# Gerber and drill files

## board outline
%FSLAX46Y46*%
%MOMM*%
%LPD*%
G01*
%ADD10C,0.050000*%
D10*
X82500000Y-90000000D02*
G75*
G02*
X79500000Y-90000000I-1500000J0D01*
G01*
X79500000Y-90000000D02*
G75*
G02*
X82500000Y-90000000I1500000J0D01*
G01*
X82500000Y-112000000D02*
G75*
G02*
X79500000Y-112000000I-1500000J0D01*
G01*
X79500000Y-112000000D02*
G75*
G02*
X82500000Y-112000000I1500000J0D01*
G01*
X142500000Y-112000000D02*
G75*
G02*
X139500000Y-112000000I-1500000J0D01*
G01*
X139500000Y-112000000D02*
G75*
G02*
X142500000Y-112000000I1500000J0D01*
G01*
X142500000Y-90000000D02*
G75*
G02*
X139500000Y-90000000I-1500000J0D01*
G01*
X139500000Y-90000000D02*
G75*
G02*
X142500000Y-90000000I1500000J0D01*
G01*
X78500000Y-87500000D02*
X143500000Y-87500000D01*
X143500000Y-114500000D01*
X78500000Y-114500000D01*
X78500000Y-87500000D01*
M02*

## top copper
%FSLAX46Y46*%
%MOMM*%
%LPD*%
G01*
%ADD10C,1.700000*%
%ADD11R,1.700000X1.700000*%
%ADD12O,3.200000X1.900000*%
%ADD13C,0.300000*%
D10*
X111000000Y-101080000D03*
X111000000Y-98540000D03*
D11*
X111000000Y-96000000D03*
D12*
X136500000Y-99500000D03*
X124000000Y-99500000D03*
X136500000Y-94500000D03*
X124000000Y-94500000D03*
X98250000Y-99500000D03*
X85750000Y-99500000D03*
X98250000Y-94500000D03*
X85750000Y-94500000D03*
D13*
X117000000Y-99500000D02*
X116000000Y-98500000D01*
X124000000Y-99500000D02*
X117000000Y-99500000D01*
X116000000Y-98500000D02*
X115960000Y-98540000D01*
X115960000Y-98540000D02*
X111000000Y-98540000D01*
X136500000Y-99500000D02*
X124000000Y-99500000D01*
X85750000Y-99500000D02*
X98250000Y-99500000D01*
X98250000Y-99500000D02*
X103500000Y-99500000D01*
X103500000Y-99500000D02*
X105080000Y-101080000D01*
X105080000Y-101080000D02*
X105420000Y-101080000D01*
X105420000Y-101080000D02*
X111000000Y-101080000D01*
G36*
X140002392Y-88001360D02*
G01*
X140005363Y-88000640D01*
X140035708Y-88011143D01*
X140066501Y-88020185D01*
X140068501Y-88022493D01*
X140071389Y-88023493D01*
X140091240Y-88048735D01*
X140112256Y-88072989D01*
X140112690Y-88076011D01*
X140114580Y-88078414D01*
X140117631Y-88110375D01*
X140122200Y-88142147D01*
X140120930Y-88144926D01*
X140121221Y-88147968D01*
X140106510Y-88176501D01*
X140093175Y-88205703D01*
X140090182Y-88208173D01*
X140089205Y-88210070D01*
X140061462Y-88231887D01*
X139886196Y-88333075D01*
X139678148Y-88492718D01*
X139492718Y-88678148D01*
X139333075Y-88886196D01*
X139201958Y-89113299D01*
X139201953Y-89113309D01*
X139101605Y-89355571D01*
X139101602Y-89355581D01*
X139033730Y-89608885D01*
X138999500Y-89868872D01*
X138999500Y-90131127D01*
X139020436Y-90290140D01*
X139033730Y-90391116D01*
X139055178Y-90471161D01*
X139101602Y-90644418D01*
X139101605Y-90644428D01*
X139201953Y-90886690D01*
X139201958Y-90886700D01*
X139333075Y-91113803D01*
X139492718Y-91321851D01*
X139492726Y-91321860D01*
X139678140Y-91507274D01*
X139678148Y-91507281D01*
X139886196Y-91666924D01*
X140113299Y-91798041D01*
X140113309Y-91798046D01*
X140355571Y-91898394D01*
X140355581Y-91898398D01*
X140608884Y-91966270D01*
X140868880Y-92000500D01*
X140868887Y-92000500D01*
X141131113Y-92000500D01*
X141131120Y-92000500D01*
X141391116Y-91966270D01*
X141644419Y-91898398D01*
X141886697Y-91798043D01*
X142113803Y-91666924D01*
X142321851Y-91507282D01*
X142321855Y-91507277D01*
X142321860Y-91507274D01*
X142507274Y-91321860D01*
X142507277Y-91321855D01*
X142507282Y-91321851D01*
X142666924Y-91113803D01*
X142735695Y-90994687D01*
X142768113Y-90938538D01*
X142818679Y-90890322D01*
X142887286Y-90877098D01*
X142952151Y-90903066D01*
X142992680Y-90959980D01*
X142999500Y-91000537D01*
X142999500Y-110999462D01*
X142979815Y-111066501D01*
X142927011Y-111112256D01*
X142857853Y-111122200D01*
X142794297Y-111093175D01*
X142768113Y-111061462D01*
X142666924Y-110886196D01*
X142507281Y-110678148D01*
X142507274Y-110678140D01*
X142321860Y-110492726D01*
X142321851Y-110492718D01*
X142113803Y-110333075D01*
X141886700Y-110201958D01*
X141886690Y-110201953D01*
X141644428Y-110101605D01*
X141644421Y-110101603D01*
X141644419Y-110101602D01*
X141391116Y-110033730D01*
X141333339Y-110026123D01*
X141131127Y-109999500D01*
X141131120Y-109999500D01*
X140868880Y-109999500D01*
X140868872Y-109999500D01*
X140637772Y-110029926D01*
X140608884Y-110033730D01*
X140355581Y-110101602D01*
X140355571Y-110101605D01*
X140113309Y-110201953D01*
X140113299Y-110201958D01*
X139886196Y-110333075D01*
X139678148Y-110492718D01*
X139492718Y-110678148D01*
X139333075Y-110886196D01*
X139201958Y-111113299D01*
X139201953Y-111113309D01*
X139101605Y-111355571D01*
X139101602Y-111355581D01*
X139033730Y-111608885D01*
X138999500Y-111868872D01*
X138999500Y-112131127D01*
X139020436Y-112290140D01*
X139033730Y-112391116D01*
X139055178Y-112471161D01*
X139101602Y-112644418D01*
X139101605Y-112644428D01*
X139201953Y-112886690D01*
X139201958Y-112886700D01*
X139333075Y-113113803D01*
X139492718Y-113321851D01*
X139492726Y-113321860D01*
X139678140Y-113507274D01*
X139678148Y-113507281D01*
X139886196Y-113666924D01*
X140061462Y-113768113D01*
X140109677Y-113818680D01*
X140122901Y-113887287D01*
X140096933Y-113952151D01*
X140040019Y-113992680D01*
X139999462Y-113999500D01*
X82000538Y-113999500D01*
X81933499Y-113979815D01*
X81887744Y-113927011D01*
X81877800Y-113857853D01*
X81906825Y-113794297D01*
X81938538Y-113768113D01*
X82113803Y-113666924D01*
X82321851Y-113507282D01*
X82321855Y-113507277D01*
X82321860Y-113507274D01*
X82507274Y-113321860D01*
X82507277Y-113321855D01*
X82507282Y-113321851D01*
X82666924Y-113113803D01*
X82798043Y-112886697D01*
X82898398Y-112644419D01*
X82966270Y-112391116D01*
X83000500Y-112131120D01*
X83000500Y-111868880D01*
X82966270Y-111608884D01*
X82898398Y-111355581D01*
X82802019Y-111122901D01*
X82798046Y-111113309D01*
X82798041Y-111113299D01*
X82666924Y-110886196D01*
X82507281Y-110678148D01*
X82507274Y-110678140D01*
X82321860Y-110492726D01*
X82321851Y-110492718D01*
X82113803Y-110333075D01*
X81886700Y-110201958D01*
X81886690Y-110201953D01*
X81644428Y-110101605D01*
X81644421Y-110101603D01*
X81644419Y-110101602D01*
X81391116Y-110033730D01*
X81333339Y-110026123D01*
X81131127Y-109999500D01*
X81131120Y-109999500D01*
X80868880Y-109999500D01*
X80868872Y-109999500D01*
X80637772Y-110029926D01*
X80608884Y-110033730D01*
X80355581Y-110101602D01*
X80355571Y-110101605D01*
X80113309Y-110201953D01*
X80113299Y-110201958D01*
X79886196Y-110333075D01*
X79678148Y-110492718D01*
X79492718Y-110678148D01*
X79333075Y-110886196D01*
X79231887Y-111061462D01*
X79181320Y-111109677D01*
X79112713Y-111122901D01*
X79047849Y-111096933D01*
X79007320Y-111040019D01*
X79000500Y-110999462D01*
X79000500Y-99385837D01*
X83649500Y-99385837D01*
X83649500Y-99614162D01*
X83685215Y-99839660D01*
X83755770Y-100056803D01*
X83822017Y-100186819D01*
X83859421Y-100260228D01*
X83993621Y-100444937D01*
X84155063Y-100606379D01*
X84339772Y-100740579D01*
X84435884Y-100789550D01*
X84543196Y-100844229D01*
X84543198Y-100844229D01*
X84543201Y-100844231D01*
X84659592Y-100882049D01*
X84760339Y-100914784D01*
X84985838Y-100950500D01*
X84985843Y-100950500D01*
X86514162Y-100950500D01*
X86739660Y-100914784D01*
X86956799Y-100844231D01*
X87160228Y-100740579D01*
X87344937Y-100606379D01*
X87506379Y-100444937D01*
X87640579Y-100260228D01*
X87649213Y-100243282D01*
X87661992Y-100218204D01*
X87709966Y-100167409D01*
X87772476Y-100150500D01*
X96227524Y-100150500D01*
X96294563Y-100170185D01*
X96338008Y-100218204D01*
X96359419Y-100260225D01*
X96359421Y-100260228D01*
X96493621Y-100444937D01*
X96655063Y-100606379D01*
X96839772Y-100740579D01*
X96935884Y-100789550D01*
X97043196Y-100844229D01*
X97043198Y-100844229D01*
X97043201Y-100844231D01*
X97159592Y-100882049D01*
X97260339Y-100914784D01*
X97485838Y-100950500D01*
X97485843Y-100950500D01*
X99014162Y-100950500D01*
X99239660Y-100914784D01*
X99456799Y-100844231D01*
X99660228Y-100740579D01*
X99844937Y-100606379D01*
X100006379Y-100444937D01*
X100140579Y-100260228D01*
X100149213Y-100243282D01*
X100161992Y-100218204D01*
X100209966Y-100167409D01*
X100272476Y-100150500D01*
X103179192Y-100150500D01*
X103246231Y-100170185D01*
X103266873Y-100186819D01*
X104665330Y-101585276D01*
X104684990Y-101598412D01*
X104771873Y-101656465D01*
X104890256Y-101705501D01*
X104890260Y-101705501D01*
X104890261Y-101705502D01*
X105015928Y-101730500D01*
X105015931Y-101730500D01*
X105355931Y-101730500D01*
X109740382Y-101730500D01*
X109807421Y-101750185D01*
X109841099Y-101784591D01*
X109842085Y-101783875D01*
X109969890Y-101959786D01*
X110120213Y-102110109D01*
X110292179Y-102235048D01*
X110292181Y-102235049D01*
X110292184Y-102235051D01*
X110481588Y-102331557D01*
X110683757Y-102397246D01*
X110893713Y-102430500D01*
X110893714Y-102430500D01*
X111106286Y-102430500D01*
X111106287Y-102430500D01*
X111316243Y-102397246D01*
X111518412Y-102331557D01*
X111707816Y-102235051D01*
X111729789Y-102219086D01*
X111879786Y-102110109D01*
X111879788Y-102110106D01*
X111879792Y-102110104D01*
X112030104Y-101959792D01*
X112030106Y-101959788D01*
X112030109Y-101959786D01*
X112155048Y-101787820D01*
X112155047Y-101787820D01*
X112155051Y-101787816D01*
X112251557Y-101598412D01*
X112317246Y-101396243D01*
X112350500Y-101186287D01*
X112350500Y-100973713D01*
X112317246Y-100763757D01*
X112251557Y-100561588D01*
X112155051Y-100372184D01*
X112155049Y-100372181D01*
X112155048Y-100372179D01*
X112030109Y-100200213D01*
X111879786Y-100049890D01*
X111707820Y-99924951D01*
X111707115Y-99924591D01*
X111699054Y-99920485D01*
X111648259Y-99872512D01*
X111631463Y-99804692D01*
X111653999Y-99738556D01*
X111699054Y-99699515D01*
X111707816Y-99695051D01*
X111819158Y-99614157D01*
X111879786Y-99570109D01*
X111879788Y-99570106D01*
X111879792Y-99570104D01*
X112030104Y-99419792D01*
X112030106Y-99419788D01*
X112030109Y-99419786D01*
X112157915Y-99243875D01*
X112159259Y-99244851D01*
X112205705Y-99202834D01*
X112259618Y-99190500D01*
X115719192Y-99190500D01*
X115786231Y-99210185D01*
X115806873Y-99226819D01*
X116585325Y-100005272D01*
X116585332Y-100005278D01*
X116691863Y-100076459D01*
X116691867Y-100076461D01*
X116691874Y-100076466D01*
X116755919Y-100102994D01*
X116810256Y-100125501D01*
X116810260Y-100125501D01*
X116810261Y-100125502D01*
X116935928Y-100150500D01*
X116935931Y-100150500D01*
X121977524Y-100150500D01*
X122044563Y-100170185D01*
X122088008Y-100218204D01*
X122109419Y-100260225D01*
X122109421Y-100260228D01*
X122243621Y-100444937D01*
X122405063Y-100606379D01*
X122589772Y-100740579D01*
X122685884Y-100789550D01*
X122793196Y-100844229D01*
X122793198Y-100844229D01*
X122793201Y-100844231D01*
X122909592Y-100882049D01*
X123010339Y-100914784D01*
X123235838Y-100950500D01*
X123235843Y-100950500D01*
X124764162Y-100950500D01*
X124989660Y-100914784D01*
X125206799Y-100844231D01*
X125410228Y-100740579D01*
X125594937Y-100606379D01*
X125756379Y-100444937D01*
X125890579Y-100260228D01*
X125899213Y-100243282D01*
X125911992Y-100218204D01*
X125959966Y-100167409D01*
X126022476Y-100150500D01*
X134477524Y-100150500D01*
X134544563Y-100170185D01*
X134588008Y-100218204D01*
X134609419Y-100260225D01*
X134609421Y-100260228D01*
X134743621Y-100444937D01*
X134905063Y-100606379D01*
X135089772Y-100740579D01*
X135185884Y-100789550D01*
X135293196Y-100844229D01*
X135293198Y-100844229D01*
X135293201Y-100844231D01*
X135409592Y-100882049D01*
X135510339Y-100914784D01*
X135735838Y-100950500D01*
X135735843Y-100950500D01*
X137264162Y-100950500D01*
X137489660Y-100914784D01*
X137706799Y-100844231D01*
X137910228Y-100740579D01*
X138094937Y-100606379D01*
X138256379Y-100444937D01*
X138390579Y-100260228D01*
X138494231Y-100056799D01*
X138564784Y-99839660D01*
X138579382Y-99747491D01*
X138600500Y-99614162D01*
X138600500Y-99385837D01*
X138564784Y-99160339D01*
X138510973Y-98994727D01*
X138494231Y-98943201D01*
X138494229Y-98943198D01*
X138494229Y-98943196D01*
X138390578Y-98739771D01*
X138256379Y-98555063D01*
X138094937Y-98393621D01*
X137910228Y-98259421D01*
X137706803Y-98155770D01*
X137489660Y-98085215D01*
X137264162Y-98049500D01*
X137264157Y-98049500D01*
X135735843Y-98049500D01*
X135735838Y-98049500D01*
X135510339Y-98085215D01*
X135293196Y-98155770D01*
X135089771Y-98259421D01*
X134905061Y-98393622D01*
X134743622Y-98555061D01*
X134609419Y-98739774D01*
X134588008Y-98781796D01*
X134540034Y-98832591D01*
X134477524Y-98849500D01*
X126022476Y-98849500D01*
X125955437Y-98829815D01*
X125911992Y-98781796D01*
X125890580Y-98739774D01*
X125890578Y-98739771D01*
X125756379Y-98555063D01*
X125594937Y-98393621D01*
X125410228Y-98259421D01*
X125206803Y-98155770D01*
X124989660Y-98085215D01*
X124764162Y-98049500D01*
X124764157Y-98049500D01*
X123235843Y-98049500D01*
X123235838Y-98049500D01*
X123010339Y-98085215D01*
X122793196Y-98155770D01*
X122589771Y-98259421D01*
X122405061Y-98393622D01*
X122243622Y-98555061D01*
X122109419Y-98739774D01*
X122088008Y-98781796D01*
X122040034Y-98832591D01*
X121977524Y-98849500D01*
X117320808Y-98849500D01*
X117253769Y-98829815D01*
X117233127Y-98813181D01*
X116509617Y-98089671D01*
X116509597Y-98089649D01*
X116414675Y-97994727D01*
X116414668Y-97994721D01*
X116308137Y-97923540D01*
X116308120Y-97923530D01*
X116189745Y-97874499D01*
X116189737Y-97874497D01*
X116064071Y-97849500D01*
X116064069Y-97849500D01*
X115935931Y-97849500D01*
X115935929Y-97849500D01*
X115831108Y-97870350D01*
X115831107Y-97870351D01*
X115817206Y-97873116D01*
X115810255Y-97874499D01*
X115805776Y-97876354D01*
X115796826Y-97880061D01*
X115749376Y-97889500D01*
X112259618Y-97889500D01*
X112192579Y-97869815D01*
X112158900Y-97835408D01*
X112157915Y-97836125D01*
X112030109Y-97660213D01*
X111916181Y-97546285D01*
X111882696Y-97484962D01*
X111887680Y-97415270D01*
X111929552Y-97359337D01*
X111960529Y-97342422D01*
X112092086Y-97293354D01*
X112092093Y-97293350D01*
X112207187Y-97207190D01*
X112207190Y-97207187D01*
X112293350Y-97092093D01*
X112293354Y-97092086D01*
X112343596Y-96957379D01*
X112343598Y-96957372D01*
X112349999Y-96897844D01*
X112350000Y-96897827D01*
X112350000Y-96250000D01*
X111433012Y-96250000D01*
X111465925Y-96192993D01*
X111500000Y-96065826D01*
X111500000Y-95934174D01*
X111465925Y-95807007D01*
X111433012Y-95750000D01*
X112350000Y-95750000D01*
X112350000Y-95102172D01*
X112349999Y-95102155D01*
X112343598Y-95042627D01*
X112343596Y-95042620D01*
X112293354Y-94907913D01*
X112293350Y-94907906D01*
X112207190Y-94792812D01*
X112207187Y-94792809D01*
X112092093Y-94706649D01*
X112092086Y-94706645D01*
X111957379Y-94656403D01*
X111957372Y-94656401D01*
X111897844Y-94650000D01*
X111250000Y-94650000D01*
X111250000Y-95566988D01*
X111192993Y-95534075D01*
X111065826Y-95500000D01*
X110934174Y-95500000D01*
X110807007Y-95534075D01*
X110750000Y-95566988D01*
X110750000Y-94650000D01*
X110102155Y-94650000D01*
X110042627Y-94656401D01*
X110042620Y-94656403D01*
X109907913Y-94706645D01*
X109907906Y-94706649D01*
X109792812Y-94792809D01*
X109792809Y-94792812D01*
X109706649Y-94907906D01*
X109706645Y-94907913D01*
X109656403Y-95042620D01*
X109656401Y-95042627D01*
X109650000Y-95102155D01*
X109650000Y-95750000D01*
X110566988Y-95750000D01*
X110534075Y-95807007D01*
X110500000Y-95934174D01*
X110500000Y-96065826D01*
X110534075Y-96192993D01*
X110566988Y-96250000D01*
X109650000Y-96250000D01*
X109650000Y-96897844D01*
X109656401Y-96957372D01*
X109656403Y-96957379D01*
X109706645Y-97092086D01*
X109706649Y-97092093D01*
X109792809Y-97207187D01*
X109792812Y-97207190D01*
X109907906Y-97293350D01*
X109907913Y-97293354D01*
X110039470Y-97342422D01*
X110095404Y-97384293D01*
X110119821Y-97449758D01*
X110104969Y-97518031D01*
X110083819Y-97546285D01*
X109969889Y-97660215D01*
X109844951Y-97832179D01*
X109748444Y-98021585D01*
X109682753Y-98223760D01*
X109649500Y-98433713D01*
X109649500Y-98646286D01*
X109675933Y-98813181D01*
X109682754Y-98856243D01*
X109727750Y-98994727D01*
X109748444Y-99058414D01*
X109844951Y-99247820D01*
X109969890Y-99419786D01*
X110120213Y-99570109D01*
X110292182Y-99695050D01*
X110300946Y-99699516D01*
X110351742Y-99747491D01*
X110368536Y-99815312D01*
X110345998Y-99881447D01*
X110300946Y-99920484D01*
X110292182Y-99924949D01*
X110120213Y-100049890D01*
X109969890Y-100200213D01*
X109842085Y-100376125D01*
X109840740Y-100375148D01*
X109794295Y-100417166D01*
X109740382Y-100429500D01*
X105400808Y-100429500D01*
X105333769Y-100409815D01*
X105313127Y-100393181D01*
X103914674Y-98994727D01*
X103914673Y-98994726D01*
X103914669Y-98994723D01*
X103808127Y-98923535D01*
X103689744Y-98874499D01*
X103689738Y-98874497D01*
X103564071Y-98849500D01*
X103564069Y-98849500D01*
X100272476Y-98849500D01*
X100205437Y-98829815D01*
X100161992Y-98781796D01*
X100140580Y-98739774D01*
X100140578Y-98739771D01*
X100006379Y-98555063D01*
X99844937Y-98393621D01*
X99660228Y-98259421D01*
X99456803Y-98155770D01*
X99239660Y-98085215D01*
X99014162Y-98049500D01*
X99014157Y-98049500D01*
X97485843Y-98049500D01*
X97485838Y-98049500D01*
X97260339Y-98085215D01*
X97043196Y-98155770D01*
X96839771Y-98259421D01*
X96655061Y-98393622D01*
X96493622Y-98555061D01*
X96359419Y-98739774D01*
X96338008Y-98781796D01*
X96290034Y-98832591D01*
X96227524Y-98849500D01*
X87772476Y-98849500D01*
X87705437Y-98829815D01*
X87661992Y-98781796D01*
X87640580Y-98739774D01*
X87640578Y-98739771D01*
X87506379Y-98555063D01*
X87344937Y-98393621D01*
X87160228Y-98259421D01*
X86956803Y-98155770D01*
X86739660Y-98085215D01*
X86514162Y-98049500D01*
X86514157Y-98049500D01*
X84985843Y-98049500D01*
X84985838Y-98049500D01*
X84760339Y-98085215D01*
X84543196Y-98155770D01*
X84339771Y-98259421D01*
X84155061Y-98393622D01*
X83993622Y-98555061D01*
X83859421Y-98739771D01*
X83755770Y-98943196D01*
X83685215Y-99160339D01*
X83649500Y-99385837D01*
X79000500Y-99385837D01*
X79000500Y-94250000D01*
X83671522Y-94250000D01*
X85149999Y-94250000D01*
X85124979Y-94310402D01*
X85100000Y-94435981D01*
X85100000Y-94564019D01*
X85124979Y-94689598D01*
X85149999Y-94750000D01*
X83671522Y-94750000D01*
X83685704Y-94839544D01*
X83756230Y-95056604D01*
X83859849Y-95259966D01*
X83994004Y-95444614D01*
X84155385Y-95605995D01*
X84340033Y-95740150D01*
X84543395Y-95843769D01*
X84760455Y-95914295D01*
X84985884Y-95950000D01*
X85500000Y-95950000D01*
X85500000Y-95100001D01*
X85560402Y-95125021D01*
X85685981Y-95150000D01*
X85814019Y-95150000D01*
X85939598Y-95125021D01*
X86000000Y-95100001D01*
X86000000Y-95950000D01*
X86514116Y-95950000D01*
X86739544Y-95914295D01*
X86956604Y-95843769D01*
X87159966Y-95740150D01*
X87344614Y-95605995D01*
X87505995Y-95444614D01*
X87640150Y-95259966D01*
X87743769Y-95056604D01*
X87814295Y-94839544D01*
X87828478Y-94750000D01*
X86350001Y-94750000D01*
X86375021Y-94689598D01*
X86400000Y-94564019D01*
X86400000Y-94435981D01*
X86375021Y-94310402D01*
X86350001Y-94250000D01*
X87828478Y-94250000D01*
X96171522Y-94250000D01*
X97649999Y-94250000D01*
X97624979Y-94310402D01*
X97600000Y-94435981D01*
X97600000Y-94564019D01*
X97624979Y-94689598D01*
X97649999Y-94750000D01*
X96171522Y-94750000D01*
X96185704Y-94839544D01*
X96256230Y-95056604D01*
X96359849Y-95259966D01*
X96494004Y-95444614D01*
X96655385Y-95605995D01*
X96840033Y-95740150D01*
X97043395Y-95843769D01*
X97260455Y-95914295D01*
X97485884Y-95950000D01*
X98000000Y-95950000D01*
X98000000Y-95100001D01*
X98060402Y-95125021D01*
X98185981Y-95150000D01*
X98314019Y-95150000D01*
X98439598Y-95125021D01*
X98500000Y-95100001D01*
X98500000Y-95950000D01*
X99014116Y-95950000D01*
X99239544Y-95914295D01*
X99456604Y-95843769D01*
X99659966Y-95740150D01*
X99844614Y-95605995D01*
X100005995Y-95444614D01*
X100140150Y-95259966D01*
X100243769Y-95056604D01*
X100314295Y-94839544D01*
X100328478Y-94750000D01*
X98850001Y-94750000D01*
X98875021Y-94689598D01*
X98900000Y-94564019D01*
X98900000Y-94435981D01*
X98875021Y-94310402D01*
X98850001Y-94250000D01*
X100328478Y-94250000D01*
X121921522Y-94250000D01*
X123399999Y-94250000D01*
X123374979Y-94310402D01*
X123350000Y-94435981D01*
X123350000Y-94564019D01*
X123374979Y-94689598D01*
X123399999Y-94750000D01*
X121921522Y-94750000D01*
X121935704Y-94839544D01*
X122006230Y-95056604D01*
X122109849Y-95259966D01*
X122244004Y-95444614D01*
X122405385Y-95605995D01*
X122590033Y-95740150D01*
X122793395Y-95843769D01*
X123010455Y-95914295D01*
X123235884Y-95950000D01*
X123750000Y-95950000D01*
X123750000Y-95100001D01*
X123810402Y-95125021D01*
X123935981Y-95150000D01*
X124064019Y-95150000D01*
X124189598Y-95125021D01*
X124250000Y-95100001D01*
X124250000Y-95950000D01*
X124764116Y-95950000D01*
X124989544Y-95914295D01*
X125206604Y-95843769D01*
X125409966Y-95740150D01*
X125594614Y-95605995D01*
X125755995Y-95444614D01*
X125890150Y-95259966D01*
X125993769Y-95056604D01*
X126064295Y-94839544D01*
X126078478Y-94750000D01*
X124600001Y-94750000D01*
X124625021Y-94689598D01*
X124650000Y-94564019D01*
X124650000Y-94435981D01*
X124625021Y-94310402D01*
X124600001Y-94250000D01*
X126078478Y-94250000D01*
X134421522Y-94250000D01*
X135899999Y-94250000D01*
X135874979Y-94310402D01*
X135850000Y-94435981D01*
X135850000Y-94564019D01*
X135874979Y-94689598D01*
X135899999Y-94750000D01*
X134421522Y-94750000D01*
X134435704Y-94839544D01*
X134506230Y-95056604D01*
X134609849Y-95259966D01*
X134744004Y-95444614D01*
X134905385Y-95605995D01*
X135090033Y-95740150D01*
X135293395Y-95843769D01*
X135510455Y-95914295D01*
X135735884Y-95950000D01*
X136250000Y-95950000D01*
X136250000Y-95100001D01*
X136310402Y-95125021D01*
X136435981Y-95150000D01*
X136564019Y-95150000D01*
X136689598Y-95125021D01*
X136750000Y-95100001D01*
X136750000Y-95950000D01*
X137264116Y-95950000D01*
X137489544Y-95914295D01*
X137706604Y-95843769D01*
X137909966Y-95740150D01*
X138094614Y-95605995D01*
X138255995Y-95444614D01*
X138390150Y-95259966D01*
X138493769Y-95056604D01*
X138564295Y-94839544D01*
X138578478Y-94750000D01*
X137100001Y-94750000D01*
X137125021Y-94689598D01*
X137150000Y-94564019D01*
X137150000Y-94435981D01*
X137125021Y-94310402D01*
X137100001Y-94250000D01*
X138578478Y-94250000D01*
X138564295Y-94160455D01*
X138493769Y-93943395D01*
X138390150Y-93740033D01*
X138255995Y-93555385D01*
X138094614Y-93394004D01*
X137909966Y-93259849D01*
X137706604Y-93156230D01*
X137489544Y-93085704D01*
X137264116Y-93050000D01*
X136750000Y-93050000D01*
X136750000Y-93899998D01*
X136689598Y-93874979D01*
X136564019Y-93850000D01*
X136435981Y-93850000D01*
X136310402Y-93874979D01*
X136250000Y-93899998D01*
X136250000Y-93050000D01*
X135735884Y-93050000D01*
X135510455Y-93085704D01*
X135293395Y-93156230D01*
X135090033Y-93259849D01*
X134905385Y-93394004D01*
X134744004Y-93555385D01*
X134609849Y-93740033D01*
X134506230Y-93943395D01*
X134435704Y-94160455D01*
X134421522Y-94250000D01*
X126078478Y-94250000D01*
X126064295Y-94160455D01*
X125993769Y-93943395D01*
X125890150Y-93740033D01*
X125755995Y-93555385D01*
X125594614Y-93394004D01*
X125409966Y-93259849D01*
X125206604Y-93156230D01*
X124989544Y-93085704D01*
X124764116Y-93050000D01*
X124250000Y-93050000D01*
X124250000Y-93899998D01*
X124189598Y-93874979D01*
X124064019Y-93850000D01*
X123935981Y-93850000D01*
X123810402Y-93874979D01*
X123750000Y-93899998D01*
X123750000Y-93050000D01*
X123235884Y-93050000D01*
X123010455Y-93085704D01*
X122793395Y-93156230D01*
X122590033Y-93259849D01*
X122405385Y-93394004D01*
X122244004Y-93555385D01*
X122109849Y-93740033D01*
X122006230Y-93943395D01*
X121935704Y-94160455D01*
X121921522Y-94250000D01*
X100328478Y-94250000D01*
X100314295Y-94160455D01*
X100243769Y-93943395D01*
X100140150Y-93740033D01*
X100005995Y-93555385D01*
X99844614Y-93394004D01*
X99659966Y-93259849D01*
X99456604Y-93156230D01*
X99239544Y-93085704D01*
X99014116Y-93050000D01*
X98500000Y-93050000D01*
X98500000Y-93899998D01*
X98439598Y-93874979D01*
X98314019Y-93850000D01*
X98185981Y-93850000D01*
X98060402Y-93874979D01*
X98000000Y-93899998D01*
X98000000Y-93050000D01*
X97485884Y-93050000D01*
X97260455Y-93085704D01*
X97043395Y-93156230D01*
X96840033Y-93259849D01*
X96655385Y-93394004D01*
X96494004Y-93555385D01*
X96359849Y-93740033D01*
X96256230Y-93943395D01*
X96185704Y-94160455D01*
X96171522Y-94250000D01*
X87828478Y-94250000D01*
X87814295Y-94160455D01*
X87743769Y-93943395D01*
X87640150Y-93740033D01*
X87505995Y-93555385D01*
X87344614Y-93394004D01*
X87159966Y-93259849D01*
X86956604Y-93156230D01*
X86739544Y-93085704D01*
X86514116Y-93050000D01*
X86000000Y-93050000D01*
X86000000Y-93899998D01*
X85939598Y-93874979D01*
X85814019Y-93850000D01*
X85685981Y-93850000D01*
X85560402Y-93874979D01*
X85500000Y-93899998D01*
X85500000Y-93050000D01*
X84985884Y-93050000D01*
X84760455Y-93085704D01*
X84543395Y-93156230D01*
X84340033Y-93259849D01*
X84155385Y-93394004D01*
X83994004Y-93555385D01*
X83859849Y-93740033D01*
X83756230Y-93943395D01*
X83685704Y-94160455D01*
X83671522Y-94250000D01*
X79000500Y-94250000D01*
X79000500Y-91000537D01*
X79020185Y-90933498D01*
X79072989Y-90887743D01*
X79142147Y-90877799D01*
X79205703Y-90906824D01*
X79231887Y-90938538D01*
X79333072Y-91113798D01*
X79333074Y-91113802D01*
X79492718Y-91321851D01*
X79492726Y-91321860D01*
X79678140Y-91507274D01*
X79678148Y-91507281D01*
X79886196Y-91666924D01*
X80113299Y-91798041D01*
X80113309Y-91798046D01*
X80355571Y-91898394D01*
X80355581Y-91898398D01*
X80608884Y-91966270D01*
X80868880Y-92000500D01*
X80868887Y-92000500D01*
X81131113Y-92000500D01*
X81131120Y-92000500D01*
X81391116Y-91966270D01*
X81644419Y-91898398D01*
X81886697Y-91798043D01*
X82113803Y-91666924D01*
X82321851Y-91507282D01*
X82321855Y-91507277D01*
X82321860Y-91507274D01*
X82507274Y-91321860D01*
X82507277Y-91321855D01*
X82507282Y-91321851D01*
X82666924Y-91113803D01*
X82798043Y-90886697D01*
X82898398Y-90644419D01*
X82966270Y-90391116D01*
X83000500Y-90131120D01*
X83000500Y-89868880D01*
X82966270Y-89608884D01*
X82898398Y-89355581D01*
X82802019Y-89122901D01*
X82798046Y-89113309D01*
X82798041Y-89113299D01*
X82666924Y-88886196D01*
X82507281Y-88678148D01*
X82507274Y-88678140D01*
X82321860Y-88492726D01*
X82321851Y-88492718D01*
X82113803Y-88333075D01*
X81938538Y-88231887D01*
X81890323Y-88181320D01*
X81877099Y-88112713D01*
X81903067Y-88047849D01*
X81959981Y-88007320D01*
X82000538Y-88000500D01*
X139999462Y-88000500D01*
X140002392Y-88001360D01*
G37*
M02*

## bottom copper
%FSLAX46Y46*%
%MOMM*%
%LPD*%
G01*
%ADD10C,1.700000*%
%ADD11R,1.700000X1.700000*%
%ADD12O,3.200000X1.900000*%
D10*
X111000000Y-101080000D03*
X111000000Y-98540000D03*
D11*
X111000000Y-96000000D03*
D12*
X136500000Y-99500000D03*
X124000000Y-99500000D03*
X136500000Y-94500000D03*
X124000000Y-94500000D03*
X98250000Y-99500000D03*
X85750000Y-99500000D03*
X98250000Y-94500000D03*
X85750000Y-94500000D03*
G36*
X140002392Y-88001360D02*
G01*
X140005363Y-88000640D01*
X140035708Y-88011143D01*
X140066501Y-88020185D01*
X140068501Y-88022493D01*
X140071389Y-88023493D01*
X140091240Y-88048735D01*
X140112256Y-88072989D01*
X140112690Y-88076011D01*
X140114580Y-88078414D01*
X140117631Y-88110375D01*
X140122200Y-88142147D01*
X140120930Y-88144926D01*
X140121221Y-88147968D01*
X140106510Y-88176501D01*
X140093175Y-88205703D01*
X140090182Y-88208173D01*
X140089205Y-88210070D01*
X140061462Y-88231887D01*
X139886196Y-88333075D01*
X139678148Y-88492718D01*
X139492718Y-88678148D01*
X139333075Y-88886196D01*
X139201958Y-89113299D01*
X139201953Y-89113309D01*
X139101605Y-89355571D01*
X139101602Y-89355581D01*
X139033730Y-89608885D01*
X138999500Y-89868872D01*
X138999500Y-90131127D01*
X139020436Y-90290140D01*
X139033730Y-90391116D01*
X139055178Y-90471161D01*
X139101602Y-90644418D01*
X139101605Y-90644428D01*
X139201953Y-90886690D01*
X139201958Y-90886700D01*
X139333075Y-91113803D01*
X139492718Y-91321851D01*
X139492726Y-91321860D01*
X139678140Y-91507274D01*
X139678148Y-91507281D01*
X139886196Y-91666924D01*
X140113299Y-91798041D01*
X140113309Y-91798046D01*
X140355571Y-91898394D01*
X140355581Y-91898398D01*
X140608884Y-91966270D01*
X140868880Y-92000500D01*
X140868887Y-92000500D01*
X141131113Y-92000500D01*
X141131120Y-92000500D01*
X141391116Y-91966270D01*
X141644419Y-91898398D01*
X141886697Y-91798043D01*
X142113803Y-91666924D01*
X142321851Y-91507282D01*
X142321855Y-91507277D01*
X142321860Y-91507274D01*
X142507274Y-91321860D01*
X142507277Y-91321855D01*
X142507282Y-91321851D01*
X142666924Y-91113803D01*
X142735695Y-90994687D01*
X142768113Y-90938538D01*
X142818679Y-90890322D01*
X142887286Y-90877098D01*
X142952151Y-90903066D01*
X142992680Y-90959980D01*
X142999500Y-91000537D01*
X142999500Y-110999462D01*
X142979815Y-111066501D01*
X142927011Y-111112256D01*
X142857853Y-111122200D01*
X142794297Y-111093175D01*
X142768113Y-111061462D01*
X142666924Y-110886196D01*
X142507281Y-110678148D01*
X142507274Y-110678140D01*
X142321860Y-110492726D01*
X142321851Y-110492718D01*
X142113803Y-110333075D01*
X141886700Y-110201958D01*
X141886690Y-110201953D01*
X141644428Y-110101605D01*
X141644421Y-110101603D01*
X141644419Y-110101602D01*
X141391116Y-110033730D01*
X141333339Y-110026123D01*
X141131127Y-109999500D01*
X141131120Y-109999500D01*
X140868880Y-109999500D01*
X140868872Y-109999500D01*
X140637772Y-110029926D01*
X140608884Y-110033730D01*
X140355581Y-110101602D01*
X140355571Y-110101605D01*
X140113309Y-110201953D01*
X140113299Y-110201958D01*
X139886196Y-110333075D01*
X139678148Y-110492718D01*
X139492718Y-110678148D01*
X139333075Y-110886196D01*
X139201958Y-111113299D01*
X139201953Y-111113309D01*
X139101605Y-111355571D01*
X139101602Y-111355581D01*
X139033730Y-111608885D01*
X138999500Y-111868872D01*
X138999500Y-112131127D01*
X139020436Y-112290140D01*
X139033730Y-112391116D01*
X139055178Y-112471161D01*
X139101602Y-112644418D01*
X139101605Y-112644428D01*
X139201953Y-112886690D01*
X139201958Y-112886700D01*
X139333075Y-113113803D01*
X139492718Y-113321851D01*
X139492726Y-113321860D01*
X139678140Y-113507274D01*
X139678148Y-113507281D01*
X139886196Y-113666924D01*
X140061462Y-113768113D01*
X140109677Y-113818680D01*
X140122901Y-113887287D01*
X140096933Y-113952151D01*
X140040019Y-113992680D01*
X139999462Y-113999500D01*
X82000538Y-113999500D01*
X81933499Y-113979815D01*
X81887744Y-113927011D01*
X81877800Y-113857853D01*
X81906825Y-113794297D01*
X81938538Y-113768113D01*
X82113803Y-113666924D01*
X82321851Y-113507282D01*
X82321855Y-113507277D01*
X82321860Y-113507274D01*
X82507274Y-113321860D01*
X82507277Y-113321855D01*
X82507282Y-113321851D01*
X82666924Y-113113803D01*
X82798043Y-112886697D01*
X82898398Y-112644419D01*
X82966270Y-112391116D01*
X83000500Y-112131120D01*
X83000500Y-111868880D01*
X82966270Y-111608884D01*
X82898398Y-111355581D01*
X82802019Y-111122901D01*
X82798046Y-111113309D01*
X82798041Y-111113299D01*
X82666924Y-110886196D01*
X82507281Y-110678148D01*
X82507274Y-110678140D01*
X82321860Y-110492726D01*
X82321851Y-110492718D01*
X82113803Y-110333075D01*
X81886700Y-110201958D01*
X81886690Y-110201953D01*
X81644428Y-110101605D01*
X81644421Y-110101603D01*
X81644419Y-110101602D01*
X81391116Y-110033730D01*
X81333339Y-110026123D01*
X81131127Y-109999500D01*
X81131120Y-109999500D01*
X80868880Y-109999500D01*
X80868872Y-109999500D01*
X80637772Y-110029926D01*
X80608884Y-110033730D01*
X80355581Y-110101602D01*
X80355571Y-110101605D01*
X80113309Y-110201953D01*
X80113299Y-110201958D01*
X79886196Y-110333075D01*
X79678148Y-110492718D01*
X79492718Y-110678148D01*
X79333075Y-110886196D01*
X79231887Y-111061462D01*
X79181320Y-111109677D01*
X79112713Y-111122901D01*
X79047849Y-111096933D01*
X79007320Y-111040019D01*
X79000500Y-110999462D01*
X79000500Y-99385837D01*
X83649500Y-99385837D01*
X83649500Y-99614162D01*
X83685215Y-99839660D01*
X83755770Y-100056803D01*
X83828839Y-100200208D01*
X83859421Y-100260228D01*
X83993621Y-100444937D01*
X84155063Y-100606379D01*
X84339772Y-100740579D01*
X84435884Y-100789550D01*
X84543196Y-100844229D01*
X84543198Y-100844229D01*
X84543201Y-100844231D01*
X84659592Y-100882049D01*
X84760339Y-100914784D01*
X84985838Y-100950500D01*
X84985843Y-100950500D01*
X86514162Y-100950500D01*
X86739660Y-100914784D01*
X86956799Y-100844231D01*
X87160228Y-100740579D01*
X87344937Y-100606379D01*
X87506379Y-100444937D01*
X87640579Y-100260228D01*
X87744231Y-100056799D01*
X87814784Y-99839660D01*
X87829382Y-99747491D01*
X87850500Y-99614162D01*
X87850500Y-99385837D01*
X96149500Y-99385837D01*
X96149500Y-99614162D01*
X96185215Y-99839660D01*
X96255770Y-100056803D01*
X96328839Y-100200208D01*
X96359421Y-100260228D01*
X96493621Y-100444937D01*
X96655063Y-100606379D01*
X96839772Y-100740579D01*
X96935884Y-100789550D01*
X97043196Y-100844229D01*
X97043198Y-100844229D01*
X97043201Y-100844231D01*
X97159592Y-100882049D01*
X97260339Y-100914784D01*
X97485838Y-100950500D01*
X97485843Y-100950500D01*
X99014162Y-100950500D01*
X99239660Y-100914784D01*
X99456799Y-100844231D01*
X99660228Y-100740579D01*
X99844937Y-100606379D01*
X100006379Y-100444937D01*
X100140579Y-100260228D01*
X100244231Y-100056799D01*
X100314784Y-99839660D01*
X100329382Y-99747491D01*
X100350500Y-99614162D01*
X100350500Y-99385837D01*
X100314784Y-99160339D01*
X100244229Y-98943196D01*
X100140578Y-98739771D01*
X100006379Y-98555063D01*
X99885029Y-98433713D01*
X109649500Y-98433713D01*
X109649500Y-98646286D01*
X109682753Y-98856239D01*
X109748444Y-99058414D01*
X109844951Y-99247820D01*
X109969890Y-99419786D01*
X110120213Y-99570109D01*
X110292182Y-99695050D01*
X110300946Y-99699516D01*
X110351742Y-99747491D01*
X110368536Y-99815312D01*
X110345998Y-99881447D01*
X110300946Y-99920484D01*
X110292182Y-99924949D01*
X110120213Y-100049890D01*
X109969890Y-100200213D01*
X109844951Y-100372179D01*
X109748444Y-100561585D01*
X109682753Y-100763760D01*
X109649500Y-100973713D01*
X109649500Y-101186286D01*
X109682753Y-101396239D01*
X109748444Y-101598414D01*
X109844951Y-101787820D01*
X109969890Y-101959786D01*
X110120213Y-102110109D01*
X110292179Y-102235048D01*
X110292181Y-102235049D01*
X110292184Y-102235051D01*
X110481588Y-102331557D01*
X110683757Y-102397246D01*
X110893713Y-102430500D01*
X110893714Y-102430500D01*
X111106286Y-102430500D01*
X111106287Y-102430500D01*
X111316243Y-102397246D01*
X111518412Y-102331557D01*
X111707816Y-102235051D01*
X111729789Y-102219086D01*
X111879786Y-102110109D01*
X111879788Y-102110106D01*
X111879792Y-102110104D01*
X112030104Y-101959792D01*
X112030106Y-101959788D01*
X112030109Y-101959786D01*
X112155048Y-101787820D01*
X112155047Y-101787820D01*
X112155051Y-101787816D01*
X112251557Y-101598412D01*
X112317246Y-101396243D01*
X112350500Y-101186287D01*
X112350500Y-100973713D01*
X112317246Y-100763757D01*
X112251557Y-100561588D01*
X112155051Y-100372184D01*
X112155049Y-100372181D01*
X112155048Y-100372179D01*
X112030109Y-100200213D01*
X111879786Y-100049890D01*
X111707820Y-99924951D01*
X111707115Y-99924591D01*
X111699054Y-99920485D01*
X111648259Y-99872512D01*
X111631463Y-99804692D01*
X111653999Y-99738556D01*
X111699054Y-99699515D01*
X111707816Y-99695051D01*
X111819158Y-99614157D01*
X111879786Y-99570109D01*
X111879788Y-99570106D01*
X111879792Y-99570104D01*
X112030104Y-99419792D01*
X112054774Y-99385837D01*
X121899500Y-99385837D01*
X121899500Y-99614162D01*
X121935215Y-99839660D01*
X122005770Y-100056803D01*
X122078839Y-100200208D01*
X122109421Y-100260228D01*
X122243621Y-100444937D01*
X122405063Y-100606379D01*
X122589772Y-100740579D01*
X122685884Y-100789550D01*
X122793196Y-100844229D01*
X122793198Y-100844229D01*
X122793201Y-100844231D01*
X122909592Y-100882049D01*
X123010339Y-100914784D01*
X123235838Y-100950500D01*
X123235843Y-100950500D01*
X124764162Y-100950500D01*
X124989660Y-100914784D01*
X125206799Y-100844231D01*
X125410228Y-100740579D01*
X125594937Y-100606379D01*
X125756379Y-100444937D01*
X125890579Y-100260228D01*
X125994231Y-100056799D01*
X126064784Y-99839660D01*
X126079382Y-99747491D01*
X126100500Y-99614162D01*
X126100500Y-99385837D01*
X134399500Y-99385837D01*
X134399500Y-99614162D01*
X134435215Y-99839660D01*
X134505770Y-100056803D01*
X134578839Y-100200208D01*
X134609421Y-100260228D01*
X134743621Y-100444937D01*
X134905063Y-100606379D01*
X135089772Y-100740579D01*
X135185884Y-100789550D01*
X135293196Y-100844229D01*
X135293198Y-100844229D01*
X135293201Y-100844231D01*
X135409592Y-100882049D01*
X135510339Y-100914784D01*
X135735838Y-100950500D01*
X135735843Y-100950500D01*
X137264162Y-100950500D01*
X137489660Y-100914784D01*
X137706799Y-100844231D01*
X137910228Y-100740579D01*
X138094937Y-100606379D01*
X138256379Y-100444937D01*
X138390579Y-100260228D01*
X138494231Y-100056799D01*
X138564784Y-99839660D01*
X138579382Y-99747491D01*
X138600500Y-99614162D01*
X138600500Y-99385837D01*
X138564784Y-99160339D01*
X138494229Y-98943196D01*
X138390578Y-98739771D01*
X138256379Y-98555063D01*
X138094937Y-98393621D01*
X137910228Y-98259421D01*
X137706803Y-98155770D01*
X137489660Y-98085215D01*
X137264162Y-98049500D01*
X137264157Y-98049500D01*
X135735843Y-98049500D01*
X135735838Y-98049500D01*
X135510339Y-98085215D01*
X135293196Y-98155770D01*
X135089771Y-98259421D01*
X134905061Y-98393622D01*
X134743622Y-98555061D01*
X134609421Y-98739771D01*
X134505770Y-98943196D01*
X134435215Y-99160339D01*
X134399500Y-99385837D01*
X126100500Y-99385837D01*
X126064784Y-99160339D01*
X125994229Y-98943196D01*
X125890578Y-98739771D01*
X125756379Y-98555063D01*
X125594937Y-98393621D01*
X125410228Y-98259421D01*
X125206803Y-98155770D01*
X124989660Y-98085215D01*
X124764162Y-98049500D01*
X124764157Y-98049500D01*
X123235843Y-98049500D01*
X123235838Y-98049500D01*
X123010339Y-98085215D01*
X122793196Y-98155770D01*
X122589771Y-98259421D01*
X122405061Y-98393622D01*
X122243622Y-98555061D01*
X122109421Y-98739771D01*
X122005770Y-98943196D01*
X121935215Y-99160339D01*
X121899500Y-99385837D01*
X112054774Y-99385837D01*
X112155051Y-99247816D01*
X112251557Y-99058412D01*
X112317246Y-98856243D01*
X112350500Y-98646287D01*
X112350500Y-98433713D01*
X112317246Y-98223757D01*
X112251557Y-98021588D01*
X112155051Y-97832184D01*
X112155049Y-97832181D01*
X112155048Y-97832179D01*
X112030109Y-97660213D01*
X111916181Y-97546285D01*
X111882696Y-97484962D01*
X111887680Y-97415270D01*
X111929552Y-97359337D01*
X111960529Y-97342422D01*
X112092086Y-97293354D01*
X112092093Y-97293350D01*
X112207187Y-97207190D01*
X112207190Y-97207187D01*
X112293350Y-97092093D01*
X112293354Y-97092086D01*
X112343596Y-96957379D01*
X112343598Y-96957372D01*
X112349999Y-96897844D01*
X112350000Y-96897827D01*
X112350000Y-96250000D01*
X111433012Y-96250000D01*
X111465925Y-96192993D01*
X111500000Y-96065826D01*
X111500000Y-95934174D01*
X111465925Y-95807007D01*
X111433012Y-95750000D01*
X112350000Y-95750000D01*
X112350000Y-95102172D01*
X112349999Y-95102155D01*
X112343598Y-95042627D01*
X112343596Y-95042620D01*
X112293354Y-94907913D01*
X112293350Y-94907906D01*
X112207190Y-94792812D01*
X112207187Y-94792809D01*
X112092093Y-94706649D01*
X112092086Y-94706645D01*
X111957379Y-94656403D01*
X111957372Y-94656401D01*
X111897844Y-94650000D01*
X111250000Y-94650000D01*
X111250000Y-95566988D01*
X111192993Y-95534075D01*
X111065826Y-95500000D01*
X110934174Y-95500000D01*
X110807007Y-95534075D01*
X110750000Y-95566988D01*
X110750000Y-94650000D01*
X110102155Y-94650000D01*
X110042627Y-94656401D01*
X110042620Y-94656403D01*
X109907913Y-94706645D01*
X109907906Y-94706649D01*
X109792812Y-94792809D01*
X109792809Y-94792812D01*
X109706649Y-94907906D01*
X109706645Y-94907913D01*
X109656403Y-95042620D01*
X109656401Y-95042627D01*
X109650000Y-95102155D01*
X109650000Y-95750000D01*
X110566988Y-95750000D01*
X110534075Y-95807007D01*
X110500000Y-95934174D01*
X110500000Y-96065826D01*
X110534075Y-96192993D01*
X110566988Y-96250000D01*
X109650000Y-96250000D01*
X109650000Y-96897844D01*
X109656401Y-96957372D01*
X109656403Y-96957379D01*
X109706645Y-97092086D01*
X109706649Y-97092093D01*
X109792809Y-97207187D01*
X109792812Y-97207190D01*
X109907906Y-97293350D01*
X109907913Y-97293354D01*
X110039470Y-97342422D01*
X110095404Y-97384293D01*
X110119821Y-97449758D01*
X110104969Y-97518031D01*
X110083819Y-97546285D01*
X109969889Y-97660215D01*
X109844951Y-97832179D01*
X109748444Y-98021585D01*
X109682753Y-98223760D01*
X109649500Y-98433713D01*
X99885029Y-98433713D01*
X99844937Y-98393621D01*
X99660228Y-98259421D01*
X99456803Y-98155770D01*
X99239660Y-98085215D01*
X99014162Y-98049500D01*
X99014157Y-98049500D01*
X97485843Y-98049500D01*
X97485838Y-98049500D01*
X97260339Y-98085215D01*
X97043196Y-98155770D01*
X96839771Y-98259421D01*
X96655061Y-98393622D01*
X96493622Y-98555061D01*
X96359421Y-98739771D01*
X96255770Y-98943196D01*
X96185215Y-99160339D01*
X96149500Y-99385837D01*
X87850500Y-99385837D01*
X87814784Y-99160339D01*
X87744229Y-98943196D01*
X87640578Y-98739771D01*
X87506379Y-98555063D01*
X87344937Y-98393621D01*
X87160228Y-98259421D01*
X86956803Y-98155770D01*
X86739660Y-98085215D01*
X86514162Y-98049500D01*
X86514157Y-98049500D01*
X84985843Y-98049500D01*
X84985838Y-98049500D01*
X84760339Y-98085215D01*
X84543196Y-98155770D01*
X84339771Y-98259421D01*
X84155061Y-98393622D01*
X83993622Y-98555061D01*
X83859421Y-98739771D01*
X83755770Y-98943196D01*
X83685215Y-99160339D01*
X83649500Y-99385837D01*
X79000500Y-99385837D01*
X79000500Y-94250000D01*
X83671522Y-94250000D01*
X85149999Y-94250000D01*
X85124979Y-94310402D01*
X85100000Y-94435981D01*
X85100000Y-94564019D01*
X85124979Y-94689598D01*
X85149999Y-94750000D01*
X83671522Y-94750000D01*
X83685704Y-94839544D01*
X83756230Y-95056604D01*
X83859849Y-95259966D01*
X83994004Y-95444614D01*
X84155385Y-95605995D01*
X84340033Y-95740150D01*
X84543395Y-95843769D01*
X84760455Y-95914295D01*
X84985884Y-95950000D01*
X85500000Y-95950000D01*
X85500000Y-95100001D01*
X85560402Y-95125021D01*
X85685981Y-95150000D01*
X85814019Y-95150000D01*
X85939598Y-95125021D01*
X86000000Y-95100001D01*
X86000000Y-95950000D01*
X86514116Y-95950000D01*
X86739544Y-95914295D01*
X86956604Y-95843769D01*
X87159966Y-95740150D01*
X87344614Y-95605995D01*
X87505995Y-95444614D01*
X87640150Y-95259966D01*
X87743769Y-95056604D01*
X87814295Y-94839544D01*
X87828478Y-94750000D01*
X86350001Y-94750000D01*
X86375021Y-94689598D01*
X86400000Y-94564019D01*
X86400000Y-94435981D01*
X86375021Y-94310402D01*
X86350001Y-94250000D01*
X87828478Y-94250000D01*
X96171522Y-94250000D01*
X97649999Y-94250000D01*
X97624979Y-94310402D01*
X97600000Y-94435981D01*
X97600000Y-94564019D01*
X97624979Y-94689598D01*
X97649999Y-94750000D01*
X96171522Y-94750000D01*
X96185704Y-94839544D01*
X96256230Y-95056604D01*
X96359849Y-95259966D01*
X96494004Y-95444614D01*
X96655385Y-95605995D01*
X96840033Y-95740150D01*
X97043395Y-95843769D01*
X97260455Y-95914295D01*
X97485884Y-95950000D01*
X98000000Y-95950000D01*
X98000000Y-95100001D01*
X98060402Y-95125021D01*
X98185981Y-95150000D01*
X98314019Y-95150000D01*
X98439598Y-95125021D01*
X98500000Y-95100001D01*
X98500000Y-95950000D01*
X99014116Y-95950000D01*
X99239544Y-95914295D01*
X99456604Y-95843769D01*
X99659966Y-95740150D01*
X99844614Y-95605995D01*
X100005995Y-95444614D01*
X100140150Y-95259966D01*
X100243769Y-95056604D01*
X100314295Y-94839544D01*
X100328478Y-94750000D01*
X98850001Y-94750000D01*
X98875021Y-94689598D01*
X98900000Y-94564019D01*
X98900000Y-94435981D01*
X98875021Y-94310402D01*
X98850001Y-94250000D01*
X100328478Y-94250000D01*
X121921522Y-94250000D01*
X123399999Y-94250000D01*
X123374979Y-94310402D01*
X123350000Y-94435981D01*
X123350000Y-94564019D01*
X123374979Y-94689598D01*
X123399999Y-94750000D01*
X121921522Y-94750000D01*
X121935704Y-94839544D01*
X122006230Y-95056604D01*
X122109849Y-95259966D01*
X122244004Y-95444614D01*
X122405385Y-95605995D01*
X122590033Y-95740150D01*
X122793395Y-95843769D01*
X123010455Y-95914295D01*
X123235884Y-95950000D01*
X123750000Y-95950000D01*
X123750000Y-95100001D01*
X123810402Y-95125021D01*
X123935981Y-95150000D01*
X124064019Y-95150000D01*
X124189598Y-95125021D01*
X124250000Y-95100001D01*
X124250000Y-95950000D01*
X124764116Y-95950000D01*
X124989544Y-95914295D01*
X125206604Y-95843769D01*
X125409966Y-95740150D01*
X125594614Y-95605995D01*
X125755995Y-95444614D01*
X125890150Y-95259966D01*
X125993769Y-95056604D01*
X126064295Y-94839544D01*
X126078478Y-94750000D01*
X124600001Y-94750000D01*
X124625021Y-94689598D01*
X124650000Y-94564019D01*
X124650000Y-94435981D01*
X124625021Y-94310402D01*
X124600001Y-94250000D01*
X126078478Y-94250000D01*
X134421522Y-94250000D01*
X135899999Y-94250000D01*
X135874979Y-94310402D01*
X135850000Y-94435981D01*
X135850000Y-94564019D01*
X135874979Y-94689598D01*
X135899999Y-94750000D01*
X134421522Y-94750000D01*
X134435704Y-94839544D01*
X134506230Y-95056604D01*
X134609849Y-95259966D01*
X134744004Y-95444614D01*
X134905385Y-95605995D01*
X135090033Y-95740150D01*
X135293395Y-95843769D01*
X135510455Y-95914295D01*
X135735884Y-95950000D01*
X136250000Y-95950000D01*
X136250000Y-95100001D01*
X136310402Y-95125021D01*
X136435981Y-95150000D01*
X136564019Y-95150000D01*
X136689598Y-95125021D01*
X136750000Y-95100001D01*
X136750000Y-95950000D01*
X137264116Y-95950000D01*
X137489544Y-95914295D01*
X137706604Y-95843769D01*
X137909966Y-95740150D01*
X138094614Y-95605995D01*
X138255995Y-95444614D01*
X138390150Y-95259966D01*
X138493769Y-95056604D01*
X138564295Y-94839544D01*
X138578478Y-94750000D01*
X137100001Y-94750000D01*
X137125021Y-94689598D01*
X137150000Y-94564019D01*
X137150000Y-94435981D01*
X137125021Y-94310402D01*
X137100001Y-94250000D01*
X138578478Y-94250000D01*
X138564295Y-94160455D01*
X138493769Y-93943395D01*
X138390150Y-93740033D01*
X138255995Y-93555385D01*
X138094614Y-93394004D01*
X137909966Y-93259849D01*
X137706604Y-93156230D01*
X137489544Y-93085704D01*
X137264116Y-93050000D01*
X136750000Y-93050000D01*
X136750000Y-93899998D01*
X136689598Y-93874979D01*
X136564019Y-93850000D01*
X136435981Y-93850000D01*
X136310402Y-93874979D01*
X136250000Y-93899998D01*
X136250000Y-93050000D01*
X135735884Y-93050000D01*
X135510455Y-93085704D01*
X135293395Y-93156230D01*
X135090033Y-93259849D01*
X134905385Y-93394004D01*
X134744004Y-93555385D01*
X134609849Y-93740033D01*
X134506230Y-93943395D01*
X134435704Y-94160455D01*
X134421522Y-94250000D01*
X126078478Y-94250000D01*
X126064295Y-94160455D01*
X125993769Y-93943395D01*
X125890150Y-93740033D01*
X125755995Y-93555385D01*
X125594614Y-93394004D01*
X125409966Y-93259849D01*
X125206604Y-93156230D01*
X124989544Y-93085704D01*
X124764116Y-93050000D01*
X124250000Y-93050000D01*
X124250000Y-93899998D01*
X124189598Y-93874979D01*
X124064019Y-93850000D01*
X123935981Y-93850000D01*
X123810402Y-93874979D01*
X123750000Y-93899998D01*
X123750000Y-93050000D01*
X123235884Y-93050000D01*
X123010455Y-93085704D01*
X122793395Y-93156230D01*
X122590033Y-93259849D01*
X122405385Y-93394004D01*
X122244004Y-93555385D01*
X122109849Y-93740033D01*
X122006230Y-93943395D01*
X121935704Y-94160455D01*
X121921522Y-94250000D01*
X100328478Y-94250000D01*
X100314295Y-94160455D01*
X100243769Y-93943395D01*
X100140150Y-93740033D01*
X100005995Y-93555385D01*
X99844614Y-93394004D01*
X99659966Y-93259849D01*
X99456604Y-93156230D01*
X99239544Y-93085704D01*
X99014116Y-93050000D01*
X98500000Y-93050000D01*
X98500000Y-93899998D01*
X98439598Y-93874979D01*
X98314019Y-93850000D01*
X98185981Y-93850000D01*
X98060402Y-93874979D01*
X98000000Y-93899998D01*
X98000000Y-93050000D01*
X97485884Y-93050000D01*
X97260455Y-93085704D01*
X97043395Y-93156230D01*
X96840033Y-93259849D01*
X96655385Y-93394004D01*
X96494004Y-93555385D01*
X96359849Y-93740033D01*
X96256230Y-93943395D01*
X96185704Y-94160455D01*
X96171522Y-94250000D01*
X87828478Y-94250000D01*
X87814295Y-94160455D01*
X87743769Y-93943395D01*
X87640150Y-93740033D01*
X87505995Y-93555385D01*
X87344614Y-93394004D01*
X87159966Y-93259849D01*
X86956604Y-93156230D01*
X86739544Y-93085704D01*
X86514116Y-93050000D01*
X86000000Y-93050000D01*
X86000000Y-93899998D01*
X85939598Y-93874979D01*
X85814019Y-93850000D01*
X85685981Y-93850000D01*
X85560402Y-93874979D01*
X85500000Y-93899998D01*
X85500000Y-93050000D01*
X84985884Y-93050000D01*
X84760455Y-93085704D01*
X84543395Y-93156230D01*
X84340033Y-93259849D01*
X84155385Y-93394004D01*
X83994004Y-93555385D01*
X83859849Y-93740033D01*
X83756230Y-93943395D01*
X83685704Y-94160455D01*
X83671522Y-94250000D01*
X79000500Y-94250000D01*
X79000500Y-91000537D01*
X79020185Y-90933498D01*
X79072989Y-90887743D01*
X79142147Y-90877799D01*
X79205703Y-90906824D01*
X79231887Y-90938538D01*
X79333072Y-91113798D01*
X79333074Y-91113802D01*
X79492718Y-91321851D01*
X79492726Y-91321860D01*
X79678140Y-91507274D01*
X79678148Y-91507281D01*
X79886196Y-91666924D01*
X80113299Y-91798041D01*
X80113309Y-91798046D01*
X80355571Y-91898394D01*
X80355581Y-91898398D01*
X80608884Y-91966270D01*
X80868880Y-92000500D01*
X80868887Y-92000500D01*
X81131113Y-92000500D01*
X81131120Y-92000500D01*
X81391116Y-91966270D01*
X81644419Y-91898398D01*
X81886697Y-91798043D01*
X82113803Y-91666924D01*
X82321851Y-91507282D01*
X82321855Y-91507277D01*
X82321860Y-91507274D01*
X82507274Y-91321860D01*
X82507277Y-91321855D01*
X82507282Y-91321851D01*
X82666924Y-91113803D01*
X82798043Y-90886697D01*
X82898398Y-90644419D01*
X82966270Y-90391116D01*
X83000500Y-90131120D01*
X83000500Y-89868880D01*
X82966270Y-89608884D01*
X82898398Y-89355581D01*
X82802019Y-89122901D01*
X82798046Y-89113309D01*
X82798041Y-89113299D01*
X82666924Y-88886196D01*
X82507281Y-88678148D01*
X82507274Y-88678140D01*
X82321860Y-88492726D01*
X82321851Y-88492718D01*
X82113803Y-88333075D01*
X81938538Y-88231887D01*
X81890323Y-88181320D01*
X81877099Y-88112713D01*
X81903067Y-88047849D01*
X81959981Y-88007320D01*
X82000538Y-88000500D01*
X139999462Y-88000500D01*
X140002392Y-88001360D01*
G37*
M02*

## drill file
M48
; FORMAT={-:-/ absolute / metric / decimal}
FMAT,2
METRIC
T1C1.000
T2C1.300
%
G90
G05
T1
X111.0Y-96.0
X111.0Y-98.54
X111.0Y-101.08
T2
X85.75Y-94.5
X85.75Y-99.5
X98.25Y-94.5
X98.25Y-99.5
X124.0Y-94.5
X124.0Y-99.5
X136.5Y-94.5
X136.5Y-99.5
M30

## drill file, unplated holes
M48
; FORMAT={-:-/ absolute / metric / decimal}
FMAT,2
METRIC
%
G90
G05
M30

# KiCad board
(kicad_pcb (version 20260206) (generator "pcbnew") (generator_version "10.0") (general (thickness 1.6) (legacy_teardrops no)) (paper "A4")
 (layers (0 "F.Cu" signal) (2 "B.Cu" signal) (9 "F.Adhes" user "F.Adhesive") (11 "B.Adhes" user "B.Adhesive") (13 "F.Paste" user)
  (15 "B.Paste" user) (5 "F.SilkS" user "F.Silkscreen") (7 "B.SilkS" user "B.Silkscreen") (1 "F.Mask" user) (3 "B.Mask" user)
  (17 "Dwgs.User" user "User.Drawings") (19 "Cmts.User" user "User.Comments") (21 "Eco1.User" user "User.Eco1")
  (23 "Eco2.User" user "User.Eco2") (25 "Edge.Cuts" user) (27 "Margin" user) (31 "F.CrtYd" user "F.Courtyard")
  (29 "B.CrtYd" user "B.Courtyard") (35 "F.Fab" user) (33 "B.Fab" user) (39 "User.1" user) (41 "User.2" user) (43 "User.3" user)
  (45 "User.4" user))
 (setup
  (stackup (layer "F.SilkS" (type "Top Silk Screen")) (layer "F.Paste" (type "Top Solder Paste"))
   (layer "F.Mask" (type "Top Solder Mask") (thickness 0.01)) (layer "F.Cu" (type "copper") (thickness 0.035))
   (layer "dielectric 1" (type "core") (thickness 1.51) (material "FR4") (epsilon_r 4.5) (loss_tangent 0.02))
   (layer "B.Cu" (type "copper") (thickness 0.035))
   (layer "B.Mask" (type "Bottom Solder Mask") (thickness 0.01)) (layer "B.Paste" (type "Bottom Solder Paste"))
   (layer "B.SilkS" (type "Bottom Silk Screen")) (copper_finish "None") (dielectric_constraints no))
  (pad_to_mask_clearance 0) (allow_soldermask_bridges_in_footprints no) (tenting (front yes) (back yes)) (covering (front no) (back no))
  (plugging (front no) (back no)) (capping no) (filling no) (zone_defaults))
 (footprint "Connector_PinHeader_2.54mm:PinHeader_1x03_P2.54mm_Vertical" (layer "F.Cu") (at 111 96)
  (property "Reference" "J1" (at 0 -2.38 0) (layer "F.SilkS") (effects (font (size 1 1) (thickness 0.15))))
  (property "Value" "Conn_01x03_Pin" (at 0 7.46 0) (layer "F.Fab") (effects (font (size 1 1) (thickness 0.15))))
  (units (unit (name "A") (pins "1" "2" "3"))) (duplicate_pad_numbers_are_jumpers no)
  (pad "1" thru_hole rect (at 0 0) (size 1.7 1.7) (drill 1) (layers "*.Cu" "*.Mask") (remove_unused_layers no) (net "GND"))
  (pad "2" thru_hole circle (at 0 2.54) (size 1.7 1.7) (drill 1) (layers "*.Cu" "*.Mask") (remove_unused_layers no) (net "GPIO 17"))
  (pad "3" thru_hole circle (at 0 5.08) (size 1.7 1.7) (drill 1) (layers "*.Cu" "*.Mask") (remove_unused_layers no) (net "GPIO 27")))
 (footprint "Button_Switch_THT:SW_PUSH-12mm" (layer "F.Cu") (at 124 94.5)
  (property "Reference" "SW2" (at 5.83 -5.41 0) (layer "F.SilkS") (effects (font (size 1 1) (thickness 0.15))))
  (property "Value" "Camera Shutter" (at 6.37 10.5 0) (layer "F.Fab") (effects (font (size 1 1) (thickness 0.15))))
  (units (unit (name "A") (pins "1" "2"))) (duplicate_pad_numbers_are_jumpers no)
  (pad "1" thru_hole oval (at 0 0) (size 3.2 1.9) (drill 1.3) (layers "*.Cu" "*.Mask") (remove_unused_layers no) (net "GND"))
  (pad "1" thru_hole oval (at 12.5 0) (size 3.2 1.9) (drill 1.3) (layers "*.Cu" "*.Mask") (remove_unused_layers no) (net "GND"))
  (pad "2" thru_hole oval (at 0 5) (size 3.2 1.9) (drill 1.3) (layers "*.Cu" "*.Mask") (remove_unused_layers no) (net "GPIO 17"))
  (pad "2" thru_hole oval (at 12.5 5) (size 3.2 1.9) (drill 1.3) (layers "*.Cu" "*.Mask") (remove_unused_layers no) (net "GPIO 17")))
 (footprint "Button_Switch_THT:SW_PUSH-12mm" (layer "F.Cu") (at 85.75 94.5)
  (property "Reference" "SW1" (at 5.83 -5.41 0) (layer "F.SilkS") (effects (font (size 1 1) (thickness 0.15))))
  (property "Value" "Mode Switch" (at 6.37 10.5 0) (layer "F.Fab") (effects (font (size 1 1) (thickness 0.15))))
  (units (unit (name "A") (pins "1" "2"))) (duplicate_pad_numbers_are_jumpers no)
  (pad "1" thru_hole oval (at 0 0) (size 3.2 1.9) (drill 1.3) (layers "*.Cu" "*.Mask") (remove_unused_layers no) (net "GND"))
  (pad "1" thru_hole oval (at 12.5 0) (size 3.2 1.9) (drill 1.3) (layers "*.Cu" "*.Mask") (remove_unused_layers no) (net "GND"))
  (pad "2" thru_hole oval (at 0 5) (size 3.2 1.9) (drill 1.3) (layers "*.Cu" "*.Mask") (remove_unused_layers no) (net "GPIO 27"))
  (pad "2" thru_hole oval (at 12.5 5) (size 3.2 1.9) (drill 1.3) (layers "*.Cu" "*.Mask") (remove_unused_layers no) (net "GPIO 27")))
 (gr_rect (start 78.5 87.5) (end 143.5 114.5) (stroke (width 0.05) (type solid)) (fill no) (layer "Edge.Cuts"))
 (gr_circle (center 81 90) (end 82.5 90) (stroke (width 0.05) (type solid)) (fill no) (layer "Edge.Cuts"))
 (gr_circle (center 81 112) (end 82.5 112) (stroke (width 0.05) (type solid)) (fill no) (layer "Edge.Cuts"))
 (gr_circle (center 141 90) (end 142.5 90) (stroke (width 0.05) (type solid)) (fill no) (layer "Edge.Cuts"))
 (gr_circle (center 141 112) (end 142.5 112) (stroke (width 0.05) (type solid)) (fill no) (layer "Edge.Cuts"))
 (segment (start 105.42 101.08) (end 111 101.08) (width 0.3) (layer "F.Cu") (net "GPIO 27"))
 (segment (start 103.5 99.5) (end 105.08 101.08) (width 0.3) (layer "F.Cu") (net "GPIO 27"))
 (segment (start 98.25 99.5) (end 103.5 99.5) (width 0.3) (layer "F.Cu") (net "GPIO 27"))
 (segment (start 85.75 99.5) (end 98.25 99.5) (width 0.3) (layer "F.Cu") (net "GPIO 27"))
 (segment (start 105.08 101.08) (end 105.42 101.08) (width 0.3) (layer "F.Cu") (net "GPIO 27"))
 (segment (start 115.96 98.54) (end 111 98.54) (width 0.3) (layer "F.Cu") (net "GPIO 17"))
 (segment (start 124 99.5) (end 117 99.5) (width 0.3) (layer "F.Cu") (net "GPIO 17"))
 (segment (start 116 98.5) (end 115.96 98.54) (width 0.3) (layer "F.Cu") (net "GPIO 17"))
 (segment (start 117 99.5) (end 116 98.5) (width 0.3) (layer "F.Cu") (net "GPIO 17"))
 (segment (start 136.5 99.5) (end 124 99.5) (width 0.3) (layer "F.Cu") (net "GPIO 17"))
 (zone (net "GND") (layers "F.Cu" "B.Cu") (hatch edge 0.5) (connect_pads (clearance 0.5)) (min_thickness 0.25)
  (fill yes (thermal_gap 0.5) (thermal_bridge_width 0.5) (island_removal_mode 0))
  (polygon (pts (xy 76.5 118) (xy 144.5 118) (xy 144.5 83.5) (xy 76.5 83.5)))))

